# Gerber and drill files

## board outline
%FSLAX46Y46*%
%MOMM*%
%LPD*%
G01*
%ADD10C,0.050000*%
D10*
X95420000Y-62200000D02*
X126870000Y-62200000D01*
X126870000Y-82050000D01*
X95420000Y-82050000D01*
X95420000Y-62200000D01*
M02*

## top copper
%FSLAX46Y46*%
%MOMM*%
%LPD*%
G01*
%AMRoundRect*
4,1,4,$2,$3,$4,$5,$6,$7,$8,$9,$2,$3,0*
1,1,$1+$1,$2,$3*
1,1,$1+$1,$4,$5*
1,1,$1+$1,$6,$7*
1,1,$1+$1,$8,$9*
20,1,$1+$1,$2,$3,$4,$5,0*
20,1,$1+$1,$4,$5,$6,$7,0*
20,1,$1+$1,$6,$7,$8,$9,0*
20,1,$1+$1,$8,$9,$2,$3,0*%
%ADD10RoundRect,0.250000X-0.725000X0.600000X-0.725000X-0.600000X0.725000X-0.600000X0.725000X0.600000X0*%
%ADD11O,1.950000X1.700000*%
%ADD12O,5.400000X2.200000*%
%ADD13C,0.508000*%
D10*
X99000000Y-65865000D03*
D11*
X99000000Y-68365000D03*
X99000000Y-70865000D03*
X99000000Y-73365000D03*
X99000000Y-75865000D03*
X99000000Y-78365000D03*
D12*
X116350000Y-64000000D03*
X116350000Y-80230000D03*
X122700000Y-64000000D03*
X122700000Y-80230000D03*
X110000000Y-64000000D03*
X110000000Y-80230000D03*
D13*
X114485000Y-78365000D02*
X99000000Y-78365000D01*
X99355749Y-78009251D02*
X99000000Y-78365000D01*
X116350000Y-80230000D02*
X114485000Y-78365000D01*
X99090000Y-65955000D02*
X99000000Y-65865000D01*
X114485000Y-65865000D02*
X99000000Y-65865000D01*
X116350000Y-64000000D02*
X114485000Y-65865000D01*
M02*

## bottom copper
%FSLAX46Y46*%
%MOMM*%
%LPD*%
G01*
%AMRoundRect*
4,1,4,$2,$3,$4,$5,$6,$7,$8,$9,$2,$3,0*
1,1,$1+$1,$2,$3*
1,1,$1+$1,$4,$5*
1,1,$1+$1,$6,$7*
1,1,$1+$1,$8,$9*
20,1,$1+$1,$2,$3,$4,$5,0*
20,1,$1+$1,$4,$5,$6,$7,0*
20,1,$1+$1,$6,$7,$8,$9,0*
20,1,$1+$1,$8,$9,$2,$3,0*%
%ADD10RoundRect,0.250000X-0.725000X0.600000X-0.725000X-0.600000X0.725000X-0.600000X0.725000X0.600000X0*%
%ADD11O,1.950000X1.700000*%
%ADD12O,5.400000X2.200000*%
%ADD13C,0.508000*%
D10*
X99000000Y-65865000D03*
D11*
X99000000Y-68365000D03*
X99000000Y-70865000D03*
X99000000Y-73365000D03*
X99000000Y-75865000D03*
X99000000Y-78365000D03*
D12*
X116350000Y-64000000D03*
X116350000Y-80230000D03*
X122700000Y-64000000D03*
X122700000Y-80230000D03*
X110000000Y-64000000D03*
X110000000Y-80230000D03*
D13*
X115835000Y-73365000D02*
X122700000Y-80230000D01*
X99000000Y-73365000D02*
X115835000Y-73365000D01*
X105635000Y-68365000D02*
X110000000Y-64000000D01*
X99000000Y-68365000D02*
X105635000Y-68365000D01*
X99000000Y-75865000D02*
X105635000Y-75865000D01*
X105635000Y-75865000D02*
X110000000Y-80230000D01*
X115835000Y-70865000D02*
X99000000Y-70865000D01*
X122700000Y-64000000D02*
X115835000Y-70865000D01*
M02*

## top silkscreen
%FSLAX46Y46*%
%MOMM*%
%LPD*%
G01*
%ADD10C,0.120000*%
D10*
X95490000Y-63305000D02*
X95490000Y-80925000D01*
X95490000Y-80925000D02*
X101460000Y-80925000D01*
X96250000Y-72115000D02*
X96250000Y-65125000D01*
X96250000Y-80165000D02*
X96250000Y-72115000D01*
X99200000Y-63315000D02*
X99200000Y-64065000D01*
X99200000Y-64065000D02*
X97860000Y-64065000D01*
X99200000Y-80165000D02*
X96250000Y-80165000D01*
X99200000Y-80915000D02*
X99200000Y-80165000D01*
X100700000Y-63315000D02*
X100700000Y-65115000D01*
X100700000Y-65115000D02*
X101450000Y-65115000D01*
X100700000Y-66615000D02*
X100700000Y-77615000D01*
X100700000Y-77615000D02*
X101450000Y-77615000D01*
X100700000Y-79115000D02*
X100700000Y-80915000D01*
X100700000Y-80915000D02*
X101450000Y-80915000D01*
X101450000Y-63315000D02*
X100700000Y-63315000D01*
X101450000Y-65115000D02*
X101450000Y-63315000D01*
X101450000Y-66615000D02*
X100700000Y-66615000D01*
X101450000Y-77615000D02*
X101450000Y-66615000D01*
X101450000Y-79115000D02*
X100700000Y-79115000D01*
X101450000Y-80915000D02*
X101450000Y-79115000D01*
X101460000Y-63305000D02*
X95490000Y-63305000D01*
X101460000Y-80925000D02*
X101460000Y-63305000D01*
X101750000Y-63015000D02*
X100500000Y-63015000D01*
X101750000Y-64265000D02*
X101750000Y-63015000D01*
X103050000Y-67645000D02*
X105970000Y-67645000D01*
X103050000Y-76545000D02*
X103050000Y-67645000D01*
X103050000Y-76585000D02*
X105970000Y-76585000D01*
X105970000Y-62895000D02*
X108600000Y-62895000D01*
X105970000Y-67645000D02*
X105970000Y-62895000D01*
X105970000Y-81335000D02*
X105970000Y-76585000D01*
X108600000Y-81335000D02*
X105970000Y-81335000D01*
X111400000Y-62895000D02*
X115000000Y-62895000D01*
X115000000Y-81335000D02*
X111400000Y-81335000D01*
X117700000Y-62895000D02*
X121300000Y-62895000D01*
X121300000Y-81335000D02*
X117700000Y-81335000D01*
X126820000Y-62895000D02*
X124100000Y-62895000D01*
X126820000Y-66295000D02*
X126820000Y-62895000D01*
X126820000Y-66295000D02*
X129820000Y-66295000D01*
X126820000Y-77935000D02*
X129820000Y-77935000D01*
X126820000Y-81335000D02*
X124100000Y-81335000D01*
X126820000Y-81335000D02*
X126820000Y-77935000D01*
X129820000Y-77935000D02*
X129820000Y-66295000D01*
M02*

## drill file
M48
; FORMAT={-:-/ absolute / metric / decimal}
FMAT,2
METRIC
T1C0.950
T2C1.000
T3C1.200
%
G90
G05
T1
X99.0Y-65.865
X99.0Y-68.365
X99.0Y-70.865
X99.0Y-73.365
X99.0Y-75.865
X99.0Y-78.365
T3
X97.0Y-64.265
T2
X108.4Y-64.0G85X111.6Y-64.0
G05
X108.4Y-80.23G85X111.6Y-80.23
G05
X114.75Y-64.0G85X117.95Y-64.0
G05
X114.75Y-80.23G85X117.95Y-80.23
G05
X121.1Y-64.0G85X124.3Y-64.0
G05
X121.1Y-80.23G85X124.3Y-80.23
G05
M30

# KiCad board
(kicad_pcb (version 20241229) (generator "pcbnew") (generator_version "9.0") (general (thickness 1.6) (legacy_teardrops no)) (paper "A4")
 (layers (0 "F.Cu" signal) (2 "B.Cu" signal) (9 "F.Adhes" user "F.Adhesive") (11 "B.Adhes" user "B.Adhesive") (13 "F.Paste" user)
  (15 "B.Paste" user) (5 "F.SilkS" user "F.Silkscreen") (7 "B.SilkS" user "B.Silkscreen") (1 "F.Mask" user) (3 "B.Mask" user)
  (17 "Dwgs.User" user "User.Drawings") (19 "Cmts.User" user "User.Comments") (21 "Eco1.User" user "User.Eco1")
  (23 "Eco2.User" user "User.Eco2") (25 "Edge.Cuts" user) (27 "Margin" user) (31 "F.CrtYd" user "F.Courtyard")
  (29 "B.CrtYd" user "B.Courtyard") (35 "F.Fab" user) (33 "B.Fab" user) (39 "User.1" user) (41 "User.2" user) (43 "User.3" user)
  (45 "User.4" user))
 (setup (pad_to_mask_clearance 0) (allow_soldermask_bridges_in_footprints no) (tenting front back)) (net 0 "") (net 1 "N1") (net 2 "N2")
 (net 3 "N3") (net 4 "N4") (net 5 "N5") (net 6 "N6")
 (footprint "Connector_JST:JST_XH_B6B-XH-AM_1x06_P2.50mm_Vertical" (layer "F.Cu") (at 99 65.865 -90)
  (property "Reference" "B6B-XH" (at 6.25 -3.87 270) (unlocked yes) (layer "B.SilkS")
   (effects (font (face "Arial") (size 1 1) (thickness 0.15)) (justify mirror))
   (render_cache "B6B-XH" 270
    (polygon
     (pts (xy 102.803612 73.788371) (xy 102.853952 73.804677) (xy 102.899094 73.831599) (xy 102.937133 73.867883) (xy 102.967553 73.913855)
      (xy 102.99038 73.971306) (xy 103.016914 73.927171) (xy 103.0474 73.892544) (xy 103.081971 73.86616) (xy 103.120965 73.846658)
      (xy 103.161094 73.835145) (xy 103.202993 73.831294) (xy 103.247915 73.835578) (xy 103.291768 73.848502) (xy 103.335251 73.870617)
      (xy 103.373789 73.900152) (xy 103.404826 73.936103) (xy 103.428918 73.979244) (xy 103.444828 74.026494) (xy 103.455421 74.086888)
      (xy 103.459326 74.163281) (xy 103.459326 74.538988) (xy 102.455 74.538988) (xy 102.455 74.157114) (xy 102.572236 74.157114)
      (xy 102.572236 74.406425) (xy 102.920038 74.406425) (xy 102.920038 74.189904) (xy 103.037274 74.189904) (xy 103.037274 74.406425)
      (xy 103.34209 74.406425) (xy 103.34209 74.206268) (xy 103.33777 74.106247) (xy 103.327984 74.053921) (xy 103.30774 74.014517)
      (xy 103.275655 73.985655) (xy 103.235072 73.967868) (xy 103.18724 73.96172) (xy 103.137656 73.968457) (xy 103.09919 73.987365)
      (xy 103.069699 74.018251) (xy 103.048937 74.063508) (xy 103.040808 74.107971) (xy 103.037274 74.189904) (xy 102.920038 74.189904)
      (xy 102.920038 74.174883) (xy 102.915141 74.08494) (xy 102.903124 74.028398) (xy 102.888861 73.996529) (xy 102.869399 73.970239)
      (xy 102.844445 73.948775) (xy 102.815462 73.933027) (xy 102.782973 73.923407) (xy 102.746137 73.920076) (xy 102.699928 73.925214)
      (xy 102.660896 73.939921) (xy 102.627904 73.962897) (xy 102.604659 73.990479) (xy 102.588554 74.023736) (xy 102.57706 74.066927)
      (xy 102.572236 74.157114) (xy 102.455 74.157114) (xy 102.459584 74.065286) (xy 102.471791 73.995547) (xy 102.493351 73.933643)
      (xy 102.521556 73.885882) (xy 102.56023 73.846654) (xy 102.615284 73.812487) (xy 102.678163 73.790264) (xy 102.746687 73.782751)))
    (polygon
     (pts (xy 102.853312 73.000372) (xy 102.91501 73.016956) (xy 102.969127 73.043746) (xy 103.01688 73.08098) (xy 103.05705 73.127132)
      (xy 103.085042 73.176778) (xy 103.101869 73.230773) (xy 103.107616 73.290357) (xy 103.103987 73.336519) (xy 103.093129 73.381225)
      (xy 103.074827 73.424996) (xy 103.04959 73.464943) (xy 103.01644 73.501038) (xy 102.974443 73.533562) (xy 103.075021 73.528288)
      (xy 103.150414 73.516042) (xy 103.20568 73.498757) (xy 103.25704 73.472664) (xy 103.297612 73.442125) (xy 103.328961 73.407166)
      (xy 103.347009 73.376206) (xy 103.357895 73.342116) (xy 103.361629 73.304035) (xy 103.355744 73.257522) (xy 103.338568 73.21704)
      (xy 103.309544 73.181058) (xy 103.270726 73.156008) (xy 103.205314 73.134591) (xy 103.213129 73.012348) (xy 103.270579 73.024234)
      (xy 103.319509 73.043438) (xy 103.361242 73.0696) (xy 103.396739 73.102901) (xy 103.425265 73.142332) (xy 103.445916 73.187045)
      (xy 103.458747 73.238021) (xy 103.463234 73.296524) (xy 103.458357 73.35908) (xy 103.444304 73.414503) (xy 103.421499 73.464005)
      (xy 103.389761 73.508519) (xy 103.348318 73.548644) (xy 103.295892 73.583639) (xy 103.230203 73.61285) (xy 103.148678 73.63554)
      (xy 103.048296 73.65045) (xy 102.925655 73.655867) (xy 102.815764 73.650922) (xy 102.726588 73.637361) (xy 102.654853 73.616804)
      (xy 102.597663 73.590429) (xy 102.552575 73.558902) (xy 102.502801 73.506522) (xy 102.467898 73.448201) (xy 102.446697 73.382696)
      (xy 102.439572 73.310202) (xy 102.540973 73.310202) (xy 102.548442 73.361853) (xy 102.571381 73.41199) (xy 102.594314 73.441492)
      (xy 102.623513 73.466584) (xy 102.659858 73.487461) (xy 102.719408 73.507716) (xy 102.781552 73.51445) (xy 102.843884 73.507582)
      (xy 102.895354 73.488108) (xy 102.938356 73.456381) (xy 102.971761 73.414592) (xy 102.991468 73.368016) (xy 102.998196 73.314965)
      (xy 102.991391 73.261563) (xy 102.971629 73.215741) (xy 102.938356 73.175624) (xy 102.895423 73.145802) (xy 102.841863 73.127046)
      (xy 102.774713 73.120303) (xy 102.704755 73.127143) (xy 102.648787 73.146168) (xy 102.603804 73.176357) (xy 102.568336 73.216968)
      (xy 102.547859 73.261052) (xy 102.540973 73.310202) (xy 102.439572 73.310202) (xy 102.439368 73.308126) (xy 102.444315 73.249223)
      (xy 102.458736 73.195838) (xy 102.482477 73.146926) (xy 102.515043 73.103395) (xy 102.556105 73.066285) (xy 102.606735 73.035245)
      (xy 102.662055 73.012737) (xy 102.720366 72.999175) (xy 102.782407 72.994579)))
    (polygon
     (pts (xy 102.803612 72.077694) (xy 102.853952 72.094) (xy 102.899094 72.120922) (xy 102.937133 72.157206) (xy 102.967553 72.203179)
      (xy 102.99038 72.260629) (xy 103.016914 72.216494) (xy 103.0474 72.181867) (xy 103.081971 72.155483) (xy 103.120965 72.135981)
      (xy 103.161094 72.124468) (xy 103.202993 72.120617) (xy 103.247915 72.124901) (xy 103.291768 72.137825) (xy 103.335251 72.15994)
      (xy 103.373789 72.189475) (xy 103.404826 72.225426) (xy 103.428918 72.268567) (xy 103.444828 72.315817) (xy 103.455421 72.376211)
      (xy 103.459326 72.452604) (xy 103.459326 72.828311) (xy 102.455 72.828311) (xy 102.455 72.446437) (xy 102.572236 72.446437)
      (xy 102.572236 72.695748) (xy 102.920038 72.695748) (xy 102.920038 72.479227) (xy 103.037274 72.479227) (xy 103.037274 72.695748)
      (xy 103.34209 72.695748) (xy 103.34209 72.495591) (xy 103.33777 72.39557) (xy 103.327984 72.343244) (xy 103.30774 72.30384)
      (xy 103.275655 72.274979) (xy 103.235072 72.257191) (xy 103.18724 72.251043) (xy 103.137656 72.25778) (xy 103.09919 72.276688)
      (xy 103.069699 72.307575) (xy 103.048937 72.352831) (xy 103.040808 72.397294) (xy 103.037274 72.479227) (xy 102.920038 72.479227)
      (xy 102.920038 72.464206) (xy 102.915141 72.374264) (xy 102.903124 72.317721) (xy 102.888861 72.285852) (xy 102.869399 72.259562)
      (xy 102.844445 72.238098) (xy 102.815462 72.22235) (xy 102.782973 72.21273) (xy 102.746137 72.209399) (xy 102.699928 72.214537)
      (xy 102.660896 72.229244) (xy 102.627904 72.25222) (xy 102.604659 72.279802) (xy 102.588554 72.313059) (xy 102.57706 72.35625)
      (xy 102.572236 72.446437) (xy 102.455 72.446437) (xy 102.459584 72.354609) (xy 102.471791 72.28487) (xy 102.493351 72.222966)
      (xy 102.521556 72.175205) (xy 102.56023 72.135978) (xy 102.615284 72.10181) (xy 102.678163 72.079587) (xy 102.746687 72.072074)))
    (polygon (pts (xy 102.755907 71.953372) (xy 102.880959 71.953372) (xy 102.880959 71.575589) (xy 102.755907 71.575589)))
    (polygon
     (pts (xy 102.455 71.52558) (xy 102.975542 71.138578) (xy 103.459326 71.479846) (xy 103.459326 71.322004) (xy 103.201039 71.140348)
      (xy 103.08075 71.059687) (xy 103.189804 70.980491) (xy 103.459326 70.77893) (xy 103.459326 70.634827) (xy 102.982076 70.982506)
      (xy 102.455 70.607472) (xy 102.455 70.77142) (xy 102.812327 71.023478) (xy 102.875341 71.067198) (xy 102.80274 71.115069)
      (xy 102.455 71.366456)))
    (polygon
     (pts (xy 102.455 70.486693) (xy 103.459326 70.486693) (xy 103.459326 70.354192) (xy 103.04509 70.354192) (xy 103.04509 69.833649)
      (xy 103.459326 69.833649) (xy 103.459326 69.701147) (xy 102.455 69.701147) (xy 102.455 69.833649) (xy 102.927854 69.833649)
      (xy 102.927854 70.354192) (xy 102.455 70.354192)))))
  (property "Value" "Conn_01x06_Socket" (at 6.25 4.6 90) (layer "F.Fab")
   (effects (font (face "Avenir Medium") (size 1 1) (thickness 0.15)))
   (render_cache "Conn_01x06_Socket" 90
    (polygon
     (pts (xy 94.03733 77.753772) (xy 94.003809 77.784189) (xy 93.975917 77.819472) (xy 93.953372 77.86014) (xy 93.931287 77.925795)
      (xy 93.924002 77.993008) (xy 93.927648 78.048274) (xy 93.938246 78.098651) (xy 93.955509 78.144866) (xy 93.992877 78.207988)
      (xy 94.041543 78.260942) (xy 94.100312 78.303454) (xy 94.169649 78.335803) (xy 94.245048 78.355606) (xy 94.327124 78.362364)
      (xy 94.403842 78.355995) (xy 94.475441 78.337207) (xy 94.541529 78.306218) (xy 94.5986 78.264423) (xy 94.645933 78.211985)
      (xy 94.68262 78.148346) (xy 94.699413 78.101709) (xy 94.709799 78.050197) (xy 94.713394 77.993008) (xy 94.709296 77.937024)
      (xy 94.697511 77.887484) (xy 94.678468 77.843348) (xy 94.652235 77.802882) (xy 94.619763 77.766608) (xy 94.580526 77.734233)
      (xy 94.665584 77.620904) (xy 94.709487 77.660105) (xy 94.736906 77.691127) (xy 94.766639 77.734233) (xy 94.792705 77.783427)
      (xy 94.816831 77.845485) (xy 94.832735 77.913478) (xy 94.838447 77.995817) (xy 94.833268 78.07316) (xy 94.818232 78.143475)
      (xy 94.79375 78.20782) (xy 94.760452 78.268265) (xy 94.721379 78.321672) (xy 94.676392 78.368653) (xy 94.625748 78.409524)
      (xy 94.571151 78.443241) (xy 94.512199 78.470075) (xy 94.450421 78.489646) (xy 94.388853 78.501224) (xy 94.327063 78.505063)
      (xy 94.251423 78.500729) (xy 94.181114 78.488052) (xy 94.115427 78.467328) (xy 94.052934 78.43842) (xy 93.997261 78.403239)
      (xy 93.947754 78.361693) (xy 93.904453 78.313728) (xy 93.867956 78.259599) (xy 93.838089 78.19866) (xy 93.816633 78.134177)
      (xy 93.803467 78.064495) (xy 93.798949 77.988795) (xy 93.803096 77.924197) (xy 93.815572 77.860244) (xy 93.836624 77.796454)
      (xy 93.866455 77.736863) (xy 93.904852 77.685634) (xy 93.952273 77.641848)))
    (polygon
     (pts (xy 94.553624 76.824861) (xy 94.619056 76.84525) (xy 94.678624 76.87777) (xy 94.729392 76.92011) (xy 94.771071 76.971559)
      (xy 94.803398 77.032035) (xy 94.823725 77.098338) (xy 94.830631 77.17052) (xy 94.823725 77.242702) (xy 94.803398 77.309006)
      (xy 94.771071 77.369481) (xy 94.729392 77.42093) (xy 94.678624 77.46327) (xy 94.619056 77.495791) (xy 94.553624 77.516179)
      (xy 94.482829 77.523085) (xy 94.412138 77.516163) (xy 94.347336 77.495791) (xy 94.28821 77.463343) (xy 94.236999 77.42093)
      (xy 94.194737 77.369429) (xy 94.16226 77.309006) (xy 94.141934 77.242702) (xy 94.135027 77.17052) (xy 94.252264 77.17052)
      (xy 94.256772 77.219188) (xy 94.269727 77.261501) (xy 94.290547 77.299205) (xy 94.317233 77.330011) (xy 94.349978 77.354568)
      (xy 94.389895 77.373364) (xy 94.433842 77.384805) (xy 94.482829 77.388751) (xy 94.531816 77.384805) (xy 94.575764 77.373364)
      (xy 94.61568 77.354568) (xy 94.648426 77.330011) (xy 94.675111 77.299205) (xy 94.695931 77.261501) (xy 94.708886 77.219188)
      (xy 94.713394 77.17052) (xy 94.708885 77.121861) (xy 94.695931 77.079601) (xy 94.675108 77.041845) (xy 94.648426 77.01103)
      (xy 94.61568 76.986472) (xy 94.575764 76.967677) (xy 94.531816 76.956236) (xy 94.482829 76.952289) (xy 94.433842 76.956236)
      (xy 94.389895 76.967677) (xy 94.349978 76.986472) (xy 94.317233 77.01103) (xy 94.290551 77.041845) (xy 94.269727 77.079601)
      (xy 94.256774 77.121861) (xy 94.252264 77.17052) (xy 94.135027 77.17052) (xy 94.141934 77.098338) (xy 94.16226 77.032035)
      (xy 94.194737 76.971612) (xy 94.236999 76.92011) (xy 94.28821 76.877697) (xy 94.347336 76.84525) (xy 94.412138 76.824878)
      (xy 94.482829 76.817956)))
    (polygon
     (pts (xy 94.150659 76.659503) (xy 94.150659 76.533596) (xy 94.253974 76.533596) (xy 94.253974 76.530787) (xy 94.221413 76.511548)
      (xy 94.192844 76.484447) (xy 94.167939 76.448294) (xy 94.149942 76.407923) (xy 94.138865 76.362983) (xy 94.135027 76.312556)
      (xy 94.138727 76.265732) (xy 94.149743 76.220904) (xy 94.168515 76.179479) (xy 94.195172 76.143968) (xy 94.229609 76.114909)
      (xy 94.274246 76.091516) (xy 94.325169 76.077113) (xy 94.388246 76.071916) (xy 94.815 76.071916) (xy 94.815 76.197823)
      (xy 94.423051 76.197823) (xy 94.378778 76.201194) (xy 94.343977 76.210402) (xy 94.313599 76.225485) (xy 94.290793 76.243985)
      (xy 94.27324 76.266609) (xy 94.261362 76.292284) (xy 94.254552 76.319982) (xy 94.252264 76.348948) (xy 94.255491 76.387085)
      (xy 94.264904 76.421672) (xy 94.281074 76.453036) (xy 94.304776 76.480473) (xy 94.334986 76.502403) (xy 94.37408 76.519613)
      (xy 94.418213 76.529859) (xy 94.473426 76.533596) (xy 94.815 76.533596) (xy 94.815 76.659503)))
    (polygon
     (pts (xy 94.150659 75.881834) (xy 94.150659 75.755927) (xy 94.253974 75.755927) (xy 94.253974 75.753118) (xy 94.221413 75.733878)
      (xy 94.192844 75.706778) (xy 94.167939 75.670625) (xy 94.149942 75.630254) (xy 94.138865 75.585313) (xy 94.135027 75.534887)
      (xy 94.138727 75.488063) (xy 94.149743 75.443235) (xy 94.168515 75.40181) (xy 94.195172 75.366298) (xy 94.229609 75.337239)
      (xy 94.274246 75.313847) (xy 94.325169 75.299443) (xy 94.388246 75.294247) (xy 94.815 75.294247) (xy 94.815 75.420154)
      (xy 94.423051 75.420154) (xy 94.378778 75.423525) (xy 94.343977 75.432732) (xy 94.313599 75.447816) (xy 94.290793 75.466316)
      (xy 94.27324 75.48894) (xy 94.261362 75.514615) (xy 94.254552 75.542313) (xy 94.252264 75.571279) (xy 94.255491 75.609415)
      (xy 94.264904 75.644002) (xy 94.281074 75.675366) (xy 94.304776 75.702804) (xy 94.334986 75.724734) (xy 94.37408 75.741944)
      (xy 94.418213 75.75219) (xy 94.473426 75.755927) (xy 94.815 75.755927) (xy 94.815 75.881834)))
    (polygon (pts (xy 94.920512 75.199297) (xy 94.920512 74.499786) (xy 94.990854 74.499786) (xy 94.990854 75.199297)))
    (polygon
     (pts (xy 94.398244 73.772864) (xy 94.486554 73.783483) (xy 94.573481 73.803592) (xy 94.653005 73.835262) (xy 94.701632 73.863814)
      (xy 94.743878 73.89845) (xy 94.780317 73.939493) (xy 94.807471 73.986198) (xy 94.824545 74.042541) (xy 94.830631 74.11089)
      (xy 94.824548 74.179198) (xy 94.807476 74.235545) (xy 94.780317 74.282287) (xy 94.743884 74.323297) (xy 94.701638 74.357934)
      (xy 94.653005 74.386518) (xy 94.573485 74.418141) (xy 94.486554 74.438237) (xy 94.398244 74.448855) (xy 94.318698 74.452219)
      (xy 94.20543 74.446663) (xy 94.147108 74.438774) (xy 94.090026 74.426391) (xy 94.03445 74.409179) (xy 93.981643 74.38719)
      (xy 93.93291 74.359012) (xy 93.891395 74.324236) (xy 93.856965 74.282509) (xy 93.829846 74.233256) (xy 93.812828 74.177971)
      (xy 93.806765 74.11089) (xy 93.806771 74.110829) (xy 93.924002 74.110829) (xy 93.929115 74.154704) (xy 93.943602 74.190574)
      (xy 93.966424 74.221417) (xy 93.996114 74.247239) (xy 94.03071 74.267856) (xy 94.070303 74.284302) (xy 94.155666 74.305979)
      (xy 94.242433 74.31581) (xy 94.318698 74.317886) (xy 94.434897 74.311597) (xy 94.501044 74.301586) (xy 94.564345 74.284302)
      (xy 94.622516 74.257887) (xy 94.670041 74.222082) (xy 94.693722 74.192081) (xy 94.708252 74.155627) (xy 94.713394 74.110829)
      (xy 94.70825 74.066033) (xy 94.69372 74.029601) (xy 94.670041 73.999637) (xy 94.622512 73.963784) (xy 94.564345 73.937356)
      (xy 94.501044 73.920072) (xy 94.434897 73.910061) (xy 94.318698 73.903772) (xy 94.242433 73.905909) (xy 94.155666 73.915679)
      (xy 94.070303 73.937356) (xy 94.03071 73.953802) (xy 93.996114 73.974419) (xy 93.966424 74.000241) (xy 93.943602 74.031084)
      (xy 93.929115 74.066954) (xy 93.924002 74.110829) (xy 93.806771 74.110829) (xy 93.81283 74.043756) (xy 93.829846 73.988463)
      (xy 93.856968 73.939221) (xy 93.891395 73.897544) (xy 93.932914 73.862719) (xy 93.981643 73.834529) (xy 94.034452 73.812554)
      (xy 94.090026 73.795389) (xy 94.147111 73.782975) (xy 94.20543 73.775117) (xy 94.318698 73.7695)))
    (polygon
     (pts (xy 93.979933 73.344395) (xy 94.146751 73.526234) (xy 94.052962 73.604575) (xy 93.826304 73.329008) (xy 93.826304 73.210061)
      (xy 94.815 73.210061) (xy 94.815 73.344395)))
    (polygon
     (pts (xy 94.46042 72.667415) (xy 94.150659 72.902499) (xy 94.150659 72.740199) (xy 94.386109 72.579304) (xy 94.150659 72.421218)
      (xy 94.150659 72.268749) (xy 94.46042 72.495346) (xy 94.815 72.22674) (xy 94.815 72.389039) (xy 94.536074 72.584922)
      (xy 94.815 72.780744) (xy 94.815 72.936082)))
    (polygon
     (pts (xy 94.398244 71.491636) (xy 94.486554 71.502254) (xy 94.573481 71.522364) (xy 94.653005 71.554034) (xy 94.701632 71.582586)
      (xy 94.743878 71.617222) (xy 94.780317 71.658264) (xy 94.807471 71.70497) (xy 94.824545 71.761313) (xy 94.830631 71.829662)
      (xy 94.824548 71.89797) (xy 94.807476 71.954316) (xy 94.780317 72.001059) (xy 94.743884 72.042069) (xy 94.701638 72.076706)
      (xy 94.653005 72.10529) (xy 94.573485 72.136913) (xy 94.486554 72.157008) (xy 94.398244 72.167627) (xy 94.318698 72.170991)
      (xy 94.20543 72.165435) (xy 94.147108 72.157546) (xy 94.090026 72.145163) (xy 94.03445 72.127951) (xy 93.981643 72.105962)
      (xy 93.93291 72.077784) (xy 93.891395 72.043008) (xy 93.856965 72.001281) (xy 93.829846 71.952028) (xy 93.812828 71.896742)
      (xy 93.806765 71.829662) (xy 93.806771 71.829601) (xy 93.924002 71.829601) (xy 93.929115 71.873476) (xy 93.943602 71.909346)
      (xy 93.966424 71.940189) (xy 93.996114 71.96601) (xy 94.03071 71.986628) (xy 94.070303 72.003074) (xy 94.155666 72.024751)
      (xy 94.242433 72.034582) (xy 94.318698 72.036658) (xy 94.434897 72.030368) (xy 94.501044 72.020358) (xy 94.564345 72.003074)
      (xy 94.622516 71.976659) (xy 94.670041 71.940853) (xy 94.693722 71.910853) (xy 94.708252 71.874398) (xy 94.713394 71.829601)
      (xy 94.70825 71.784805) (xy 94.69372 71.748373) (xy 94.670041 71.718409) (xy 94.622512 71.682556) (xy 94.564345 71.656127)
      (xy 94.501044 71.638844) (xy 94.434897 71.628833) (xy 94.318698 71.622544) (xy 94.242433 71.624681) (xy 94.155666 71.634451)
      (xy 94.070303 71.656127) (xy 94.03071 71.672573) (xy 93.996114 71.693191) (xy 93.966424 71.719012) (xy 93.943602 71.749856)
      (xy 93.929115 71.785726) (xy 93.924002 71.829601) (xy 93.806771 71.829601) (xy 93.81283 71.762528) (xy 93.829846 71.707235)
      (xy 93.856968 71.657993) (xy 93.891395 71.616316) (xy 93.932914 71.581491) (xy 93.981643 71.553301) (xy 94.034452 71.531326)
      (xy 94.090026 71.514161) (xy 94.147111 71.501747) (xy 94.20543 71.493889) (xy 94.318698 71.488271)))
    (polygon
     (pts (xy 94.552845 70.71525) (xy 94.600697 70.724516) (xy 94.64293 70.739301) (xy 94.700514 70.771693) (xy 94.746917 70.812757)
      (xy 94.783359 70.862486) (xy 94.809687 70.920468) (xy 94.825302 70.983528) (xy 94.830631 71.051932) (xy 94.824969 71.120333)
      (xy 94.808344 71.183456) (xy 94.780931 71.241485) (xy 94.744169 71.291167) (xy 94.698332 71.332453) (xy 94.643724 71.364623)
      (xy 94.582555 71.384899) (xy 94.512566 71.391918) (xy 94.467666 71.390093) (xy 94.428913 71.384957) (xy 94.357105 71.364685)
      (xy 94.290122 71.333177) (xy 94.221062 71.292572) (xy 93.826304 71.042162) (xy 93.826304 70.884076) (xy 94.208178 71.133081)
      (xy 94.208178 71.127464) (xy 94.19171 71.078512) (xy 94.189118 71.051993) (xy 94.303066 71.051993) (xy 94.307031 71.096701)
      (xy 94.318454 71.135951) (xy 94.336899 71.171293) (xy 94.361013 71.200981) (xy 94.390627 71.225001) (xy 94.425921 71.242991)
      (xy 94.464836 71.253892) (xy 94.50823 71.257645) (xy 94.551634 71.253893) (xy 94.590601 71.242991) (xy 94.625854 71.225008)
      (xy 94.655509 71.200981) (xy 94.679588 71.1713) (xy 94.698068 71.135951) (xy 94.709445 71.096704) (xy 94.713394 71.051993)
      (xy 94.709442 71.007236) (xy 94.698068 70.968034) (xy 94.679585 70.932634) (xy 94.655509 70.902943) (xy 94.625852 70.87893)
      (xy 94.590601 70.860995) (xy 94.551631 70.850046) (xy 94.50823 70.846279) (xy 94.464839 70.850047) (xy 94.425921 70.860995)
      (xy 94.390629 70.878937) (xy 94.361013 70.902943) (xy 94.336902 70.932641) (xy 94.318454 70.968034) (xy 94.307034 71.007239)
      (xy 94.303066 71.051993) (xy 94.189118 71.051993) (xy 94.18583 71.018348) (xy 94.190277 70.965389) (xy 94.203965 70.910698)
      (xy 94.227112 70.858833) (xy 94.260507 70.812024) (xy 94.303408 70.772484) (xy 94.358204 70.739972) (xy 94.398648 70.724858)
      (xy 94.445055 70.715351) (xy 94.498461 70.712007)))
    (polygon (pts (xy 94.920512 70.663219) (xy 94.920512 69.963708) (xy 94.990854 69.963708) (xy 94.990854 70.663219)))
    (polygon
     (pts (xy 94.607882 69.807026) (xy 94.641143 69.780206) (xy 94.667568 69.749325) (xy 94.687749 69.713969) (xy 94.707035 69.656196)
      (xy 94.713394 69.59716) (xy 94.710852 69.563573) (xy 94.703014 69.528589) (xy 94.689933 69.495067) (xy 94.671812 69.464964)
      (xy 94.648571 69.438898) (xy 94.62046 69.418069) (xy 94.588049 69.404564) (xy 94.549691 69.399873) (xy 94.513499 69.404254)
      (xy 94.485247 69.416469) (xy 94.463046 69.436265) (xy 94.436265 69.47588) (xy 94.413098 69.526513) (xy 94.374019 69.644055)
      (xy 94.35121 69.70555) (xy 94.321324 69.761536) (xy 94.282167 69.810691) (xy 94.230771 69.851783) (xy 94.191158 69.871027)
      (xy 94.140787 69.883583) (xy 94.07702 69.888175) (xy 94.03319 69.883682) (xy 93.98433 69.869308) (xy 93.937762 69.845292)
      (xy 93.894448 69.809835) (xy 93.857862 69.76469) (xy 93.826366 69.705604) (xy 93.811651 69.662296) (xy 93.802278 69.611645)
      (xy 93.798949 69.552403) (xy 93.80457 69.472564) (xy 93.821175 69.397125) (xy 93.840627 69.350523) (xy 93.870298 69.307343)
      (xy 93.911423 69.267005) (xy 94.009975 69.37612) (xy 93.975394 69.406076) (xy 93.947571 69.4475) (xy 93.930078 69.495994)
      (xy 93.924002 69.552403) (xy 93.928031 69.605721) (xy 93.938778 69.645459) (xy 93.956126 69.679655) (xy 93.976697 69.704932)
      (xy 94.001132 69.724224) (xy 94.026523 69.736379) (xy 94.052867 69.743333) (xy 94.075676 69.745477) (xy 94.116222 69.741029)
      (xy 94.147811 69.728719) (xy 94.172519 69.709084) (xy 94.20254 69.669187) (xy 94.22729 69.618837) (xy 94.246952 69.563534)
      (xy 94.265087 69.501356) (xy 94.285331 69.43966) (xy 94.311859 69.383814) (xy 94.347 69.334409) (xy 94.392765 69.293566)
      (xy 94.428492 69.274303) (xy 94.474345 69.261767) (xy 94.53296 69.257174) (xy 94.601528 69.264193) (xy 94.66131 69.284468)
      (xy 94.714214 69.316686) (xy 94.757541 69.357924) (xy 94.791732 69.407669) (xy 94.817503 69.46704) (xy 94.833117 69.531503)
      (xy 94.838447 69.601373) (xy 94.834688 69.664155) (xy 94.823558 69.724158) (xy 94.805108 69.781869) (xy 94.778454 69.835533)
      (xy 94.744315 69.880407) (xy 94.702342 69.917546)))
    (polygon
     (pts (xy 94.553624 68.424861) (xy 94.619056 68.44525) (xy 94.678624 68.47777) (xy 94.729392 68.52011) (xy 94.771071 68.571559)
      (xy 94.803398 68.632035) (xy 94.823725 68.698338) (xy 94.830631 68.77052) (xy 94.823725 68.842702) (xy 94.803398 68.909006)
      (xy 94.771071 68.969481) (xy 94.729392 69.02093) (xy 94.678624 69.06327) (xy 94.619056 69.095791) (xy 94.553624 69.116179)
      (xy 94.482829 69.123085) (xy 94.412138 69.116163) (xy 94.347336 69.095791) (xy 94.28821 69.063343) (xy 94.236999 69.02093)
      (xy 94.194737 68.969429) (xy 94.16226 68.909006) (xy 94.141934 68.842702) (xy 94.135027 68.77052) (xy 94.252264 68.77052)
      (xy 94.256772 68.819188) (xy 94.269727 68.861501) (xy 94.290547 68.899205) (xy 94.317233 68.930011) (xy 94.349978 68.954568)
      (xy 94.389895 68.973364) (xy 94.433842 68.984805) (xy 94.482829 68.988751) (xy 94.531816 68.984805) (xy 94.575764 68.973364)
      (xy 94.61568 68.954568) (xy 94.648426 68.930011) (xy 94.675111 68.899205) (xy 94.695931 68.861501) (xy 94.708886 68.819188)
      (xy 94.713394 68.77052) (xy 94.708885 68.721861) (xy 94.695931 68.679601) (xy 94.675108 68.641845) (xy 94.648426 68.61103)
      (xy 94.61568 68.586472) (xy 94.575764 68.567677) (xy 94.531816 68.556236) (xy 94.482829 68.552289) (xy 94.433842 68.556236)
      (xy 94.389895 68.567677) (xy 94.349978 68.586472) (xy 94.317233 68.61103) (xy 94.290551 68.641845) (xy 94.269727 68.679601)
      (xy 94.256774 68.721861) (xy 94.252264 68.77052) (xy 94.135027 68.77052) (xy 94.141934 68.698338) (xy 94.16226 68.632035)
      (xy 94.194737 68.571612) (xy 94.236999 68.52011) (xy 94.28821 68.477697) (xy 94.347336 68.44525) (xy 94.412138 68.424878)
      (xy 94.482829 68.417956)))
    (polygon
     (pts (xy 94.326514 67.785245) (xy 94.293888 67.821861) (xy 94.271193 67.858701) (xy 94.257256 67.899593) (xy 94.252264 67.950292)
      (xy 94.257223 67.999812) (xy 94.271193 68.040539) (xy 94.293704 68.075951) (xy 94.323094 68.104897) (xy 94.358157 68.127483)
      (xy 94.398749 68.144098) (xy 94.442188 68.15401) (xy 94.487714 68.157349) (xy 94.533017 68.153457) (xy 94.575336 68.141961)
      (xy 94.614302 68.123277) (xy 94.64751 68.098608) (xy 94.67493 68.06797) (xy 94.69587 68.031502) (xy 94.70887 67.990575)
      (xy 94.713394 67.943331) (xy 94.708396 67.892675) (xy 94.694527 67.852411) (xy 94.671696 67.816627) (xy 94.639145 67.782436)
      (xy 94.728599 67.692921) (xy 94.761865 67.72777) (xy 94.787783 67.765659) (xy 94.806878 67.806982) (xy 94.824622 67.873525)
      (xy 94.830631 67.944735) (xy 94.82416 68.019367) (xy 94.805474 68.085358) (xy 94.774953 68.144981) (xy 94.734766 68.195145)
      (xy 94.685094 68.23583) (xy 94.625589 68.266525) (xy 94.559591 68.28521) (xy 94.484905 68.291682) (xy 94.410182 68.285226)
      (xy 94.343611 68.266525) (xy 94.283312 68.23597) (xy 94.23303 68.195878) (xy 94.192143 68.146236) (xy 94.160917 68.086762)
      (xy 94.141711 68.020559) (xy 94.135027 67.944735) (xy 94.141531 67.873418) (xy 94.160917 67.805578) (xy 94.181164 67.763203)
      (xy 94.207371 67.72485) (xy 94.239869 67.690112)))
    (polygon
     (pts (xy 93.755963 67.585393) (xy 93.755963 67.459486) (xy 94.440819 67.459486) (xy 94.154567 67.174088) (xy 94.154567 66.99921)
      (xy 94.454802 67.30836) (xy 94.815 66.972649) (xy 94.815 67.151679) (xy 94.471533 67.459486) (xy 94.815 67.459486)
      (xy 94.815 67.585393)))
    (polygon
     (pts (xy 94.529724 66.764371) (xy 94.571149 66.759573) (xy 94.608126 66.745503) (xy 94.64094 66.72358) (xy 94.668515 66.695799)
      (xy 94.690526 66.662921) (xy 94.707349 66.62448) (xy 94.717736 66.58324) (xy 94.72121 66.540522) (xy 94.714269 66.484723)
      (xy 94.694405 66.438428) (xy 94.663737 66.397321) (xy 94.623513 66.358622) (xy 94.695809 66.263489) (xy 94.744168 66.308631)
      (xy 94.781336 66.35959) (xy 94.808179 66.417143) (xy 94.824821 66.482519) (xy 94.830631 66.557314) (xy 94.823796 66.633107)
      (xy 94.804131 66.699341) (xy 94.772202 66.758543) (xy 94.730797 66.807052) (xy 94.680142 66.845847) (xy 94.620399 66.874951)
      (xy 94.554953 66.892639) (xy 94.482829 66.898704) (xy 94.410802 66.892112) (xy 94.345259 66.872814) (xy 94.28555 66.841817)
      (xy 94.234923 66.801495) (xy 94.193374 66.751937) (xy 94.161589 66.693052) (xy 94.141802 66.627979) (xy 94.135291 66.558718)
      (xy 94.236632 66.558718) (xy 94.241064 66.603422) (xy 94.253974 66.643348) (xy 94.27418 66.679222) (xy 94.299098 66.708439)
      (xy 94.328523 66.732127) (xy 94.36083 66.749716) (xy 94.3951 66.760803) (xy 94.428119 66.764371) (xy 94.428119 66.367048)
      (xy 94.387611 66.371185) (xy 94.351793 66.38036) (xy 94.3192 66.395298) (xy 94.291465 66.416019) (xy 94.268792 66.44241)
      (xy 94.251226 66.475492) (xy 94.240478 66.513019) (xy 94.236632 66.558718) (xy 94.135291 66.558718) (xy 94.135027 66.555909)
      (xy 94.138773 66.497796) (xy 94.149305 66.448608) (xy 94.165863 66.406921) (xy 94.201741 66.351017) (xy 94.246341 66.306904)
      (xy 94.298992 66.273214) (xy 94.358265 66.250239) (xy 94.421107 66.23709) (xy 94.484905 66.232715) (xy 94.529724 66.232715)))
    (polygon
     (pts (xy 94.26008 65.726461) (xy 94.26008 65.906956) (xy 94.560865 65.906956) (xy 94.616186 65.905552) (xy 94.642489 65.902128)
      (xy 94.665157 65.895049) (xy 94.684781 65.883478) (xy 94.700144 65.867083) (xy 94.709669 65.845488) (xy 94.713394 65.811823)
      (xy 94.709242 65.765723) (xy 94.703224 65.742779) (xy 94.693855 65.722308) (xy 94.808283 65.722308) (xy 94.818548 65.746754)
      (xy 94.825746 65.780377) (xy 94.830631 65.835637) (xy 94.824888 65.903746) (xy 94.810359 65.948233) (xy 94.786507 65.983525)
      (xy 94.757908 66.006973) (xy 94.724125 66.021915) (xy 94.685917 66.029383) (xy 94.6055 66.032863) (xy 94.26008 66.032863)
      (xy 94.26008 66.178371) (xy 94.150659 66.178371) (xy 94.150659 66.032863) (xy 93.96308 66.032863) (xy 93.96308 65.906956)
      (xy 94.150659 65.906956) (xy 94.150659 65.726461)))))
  (fp_line (start -2.56 3.51) (end 15.06 3.51) (stroke (width 0.12) (type solid)) (layer "F.SilkS"))
  (fp_line (start 15.06 3.51) (end 15.06 -2.46) (stroke (width 0.12) (type solid)) (layer "F.SilkS"))
  (fp_line (start 6.25 2.75) (end -0.74 2.75) (stroke (width 0.12) (type solid)) (layer "F.SilkS"))
  (fp_line (start 14.3 2.75) (end 6.25 2.75) (stroke (width 0.12) (type solid)) (layer "F.SilkS"))
  (fp_line (start -2.55 -0.2) (end -1.8 -0.2) (stroke (width 0.12) (type solid)) (layer "F.SilkS"))
  (fp_line (start -1.8 -0.2) (end -1.8 1.14) (stroke (width 0.12) (type solid)) (layer "F.SilkS"))
  (fp_line (start 14.3 -0.2) (end 14.3 2.75) (stroke (width 0.12) (type solid)) (layer "F.SilkS"))
  (fp_line (start 15.05 -0.2) (end 14.3 -0.2) (stroke (width 0.12) (type solid)) (layer "F.SilkS"))
  (fp_line (start -2.55 -1.7) (end -0.75 -1.7) (stroke (width 0.12) (type solid)) (layer "F.SilkS"))
  (fp_line (start -0.75 -1.7) (end -0.75 -2.45) (stroke (width 0.12) (type solid)) (layer "F.SilkS"))
  (fp_line (start 0.75 -1.7) (end 11.75 -1.7) (stroke (width 0.12) (type solid)) (layer "F.SilkS"))
  (fp_line (start 11.75 -1.7) (end 11.75 -2.45) (stroke (width 0.12) (type solid)) (layer "F.SilkS"))
  (fp_line (start 13.25 -1.7) (end 15.05 -1.7) (stroke (width 0.12) (type solid)) (layer "F.SilkS"))
  (fp_line (start 15.05 -1.7) (end 15.05 -2.45) (stroke (width 0.12) (type solid)) (layer "F.SilkS"))
  (fp_line (start -2.55 -2.45) (end -2.55 -1.7) (stroke (width 0.12) (type solid)) (layer "F.SilkS"))
  (fp_line (start -0.75 -2.45) (end -2.55 -2.45) (stroke (width 0.12) (type solid)) (layer "F.SilkS"))
  (fp_line (start 0.75 -2.45) (end 0.75 -1.7) (stroke (width 0.12) (type solid)) (layer "F.SilkS"))
  (fp_line (start 11.75 -2.45) (end 0.75 -2.45) (stroke (width 0.12) (type solid)) (layer "F.SilkS"))
  (fp_line (start 13.25 -2.45) (end 13.25 -1.7) (stroke (width 0.12) (type solid)) (layer "F.SilkS"))
  (fp_line (start 15.05 -2.45) (end 13.25 -2.45) (stroke (width 0.12) (type solid)) (layer "F.SilkS"))
  (fp_line (start -2.56 -2.46) (end -2.56 3.51) (stroke (width 0.12) (type solid)) (layer "F.SilkS"))
  (fp_line (start 15.06 -2.46) (end -2.56 -2.46) (stroke (width 0.12) (type solid)) (layer "F.SilkS"))
  (fp_line (start -2.85 -2.75) (end -2.85 -1.5) (stroke (width 0.12) (type solid)) (layer "F.SilkS"))
  (fp_line (start -1.6 -2.75) (end -2.85 -2.75) (stroke (width 0.12) (type solid)) (layer "F.SilkS"))
  (pad "" np_thru_hole circle (at -1.6 2 270) (size 1.2 1.2) (drill 1.2) (layers "*.Cu" "*.Mask"))
  (pad "1" thru_hole roundrect (at 0 0 270) (size 1.7 1.95) (drill 0.95) (layers "*.Cu" "*.Mask") (remove_unused_layers no)
   (roundrect_rratio 0.147059) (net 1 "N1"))
  (pad "2" thru_hole oval (at 2.5 0 270) (size 1.7 1.95) (drill 0.95) (layers "*.Cu" "*.Mask") (remove_unused_layers no) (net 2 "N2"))
  (pad "3" thru_hole oval (at 5 0 270) (size 1.7 1.95) (drill 0.95) (layers "*.Cu" "*.Mask") (remove_unused_layers no) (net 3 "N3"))
  (pad "4" thru_hole oval (at 7.5 0 270) (size 1.7 1.95) (drill 0.95) (layers "*.Cu" "*.Mask") (remove_unused_layers no) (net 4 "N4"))
  (pad "5" thru_hole oval (at 10 0 270) (size 1.7 1.95) (drill 0.95) (layers "*.Cu" "*.Mask") (remove_unused_layers no) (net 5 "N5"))
  (pad "6" thru_hole oval (at 12.5 0 270) (size 1.7 1.95) (drill 0.95) (layers "*.Cu" "*.Mask") (remove_unused_layers no) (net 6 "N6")))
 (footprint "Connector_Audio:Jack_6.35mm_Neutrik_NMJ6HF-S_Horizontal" (layer "F.Cu") (at 110 64)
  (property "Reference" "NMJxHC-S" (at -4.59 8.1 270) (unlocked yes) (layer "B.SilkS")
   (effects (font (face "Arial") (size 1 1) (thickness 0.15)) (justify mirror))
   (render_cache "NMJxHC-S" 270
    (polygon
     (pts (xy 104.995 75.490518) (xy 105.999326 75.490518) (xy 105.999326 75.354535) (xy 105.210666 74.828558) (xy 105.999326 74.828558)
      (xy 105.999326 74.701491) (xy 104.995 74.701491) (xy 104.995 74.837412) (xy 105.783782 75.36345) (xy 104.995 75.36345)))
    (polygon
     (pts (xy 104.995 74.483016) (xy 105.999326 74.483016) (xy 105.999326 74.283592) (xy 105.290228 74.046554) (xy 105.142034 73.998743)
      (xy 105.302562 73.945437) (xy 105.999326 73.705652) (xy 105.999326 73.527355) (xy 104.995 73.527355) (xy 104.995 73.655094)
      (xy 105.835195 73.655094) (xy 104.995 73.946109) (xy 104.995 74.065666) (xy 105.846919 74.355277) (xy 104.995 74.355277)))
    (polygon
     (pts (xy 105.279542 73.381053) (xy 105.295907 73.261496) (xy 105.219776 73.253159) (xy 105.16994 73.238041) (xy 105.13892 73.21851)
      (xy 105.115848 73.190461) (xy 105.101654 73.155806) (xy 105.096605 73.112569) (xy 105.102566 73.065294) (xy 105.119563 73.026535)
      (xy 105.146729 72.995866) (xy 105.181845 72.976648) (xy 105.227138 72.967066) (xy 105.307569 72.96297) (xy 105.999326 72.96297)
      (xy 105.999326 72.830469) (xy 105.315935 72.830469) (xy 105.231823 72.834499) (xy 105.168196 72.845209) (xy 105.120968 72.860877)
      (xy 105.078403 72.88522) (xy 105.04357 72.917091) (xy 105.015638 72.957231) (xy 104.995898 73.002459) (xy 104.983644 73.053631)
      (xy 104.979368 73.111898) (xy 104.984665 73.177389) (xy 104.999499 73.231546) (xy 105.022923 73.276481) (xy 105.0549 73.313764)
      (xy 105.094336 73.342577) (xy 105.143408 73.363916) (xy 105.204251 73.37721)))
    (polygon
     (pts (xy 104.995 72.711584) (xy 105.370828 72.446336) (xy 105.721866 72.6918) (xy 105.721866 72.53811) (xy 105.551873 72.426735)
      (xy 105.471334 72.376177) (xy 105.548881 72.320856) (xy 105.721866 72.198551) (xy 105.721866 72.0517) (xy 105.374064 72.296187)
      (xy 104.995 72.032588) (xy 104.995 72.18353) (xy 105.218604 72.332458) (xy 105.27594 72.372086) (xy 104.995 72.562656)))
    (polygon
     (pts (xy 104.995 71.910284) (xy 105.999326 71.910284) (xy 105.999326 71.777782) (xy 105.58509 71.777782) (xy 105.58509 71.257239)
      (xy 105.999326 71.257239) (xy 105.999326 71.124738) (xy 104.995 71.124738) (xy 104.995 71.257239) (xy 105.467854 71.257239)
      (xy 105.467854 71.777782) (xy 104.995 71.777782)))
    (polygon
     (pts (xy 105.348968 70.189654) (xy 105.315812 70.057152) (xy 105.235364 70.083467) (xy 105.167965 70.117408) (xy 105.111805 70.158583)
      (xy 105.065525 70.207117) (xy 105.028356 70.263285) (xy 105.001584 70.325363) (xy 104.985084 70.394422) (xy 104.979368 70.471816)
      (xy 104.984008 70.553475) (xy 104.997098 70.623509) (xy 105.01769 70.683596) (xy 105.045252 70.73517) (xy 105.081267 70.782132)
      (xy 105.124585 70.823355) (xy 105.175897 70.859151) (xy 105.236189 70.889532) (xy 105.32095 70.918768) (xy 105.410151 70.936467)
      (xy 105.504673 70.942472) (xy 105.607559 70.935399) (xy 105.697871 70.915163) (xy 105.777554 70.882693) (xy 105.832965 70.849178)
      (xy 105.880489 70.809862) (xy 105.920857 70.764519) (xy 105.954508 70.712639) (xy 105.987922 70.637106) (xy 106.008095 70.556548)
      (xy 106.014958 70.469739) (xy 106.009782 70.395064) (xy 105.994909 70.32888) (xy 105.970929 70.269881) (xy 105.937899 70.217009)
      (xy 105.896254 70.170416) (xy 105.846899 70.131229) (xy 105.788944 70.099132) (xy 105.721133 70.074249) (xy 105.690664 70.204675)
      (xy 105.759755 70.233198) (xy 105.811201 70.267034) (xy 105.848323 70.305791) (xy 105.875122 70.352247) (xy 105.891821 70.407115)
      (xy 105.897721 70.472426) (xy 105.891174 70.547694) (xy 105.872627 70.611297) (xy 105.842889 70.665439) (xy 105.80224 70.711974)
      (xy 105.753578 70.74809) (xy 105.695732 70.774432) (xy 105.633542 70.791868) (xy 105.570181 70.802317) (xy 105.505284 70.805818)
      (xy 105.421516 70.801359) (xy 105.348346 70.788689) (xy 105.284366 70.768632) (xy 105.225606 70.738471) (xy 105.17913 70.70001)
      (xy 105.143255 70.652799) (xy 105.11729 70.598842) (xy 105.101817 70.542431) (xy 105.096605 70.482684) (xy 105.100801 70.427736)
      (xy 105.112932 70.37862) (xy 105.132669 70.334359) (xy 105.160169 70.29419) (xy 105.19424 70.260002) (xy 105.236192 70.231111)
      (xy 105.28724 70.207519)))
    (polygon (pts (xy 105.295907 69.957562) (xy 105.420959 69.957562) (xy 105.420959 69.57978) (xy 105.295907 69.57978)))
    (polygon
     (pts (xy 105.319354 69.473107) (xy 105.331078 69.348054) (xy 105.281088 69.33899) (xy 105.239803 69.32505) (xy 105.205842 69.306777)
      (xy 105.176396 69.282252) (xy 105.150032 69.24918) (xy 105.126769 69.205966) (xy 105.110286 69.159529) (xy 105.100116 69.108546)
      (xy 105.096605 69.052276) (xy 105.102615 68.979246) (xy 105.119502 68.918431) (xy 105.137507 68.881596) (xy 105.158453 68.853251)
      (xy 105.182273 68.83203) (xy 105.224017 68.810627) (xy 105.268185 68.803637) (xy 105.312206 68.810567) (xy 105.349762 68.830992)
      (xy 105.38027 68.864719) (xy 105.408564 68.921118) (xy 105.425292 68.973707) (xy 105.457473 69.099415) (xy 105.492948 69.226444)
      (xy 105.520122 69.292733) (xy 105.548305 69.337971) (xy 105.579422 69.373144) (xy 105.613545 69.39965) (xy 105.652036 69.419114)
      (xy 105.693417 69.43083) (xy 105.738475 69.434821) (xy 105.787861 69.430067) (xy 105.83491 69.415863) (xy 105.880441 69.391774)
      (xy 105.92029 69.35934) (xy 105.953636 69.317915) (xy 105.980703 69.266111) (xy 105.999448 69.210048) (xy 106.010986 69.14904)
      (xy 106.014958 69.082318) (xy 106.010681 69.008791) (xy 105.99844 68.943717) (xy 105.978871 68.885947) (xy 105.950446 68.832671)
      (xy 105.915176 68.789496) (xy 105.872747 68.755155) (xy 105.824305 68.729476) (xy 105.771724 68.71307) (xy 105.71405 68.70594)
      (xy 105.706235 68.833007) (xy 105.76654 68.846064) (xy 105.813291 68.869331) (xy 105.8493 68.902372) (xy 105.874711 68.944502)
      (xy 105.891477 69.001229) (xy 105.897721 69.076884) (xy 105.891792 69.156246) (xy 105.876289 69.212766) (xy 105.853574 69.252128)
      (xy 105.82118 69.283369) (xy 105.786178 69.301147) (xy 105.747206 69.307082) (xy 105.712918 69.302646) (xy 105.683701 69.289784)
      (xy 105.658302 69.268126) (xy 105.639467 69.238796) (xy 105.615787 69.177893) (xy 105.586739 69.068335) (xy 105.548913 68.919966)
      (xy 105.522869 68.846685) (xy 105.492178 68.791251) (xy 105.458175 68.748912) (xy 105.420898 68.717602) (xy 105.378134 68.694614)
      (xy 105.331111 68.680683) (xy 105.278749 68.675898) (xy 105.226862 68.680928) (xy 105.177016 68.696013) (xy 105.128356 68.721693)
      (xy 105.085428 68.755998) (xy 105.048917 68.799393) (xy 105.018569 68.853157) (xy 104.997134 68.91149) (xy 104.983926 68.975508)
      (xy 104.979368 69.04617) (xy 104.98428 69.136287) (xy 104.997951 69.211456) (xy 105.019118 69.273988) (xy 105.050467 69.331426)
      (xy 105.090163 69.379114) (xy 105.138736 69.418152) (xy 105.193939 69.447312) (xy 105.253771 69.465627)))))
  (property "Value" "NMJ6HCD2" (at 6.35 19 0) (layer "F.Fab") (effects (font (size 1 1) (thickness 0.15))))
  (fp_line (start -6.95 3.645) (end -4.03 3.645) (stroke (width 0.12) (type solid)) (layer "F.SilkS"))
  (fp_line (start -6.95 12.545) (end -6.95 3.645) (stroke (width 0.12) (type solid)) (layer "F.SilkS"))
  (fp_line (start -6.95 12.585) (end -4.03 12.585) (stroke (width 0.12) (type solid)) (layer "F.SilkS"))
  (fp_line (start -4.03 -1.105) (end -1.4 -1.105) (stroke (width 0.12) (type solid)) (layer "F.SilkS"))
  (fp_line (start -4.03 3.645) (end -4.03 -1.105) (stroke (width 0.12) (type solid)) (layer "F.SilkS"))
  (fp_line (start -4.03 17.335) (end -4.03 12.585) (stroke (width 0.12) (type solid)) (layer "F.SilkS"))
  (fp_line (start -1.4 17.335) (end -4.03 17.335) (stroke (width 0.12) (type solid)) (layer "F.SilkS"))
  (fp_line (start 1.4 -1.105) (end 5 -1.105) (stroke (width 0.12) (type solid)) (layer "F.SilkS"))
  (fp_line (start 5 17.335) (end 1.4 17.335) (stroke (width 0.12) (type solid)) (layer "F.SilkS"))
  (fp_line (start 7.7 -1.105) (end 11.3 -1.105) (stroke (width 0.12) (type solid)) (layer "F.SilkS"))
  (fp_line (start 11.3 17.335) (end 7.7 17.335) (stroke (width 0.12) (type solid)) (layer "F.SilkS"))
  (fp_line (start 16.82 -1.105) (end 14.1 -1.105) (stroke (width 0.12) (type solid)) (layer "F.SilkS"))
  (fp_line (start 16.82 2.295) (end 16.82 -1.105) (stroke (width 0.12) (type solid)) (layer "F.SilkS"))
  (fp_line (start 16.82 2.295) (end 19.82 2.295) (stroke (width 0.12) (type solid)) (layer "F.SilkS"))
  (fp_line (start 16.82 13.935) (end 19.82 13.935) (stroke (width 0.12) (type solid)) (layer "F.SilkS"))
  (fp_line (start 16.82 17.335) (end 14.1 17.335) (stroke (width 0.12) (type solid)) (layer "F.SilkS"))
  (fp_line (start 16.82 17.335) (end 16.82 13.935) (stroke (width 0.12) (type solid)) (layer "F.SilkS"))
  (fp_line (start 19.82 13.935) (end 19.82 2.295) (stroke (width 0.12) (type solid)) (layer "F.SilkS"))
  (pad "R" thru_hole oval (at 6.35 0) (size 5.4 2.2) (drill oval 4.2 1) (layers "*.Cu" "*.Mask") (remove_unused_layers no) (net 1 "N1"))
  (pad "RN" thru_hole oval (at 6.35 16.23) (size 5.4 2.2) (drill oval 4.2 1) (layers "*.Cu" "*.Mask") (remove_unused_layers no) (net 6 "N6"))
  (pad "S" thru_hole oval (at 12.7 0) (size 5.4 2.2) (drill oval 4.2 1) (layers "*.Cu" "*.Mask") (remove_unused_layers no) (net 3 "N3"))
  (pad "SN" thru_hole oval (at 12.7 16.23) (size 5.4 2.2) (drill oval 4.2 1) (layers "*.Cu" "*.Mask") (remove_unused_layers no) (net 4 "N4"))
  (pad "T" thru_hole oval (at 0 0) (size 5.4 2.2) (drill oval 4.2 1) (layers "*.Cu" "*.Mask") (remove_unused_layers no) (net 2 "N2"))
  (pad "TN" thru_hole oval (at 0 16.23) (size 5.4 2.2) (drill oval 4.2 1) (layers "*.Cu" "*.Mask") (remove_unused_layers no) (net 5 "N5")))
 (gr_rect (start 95.42 62.2) (end 126.87 82.05) (stroke (width 0.05) (type solid)) (fill no) (layer "Edge.Cuts"))
 (segment (start 115.835 73.365) (end 122.7 80.23) (width 0.508) (layer "B.Cu") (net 4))
 (segment (start 99 73.365) (end 115.835 73.365) (width 0.508) (layer "B.Cu") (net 4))
 (segment (start 114.485 78.365) (end 99 78.365) (width 0.508) (layer "F.Cu") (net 6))
 (segment (start 99.355749 78.009251) (end 99 78.365) (width 0.508) (layer "F.Cu") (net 6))
 (segment (start 116.35 80.23) (end 114.485 78.365) (width 0.508) (layer "F.Cu") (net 6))
 (segment (start 105.635 68.365) (end 110 64) (width 0.508) (layer "B.Cu") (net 2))
 (segment (start 99 68.365) (end 105.635 68.365) (width 0.508) (layer "B.Cu") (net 2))
 (segment (start 99.09 65.955) (end 99 65.865) (width 0.508) (layer "F.Cu") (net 1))
 (segment (start 114.485 65.865) (end 99 65.865) (width 0.508) (layer "F.Cu") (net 1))
 (segment (start 116.35 64) (end 114.485 65.865) (width 0.508) (layer "F.Cu") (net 1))
 (segment (start 99 75.865) (end 105.635 75.865) (width 0.508) (layer "B.Cu") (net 5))
 (segment (start 105.635 75.865) (end 110 80.23) (width 0.508) (layer "B.Cu") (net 5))
 (segment (start 115.835 70.865) (end 99 70.865) (width 0.508) (layer "B.Cu") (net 3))
 (segment (start 122.7 64) (end 115.835 70.865) (width 0.508) (layer "B.Cu") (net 3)))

